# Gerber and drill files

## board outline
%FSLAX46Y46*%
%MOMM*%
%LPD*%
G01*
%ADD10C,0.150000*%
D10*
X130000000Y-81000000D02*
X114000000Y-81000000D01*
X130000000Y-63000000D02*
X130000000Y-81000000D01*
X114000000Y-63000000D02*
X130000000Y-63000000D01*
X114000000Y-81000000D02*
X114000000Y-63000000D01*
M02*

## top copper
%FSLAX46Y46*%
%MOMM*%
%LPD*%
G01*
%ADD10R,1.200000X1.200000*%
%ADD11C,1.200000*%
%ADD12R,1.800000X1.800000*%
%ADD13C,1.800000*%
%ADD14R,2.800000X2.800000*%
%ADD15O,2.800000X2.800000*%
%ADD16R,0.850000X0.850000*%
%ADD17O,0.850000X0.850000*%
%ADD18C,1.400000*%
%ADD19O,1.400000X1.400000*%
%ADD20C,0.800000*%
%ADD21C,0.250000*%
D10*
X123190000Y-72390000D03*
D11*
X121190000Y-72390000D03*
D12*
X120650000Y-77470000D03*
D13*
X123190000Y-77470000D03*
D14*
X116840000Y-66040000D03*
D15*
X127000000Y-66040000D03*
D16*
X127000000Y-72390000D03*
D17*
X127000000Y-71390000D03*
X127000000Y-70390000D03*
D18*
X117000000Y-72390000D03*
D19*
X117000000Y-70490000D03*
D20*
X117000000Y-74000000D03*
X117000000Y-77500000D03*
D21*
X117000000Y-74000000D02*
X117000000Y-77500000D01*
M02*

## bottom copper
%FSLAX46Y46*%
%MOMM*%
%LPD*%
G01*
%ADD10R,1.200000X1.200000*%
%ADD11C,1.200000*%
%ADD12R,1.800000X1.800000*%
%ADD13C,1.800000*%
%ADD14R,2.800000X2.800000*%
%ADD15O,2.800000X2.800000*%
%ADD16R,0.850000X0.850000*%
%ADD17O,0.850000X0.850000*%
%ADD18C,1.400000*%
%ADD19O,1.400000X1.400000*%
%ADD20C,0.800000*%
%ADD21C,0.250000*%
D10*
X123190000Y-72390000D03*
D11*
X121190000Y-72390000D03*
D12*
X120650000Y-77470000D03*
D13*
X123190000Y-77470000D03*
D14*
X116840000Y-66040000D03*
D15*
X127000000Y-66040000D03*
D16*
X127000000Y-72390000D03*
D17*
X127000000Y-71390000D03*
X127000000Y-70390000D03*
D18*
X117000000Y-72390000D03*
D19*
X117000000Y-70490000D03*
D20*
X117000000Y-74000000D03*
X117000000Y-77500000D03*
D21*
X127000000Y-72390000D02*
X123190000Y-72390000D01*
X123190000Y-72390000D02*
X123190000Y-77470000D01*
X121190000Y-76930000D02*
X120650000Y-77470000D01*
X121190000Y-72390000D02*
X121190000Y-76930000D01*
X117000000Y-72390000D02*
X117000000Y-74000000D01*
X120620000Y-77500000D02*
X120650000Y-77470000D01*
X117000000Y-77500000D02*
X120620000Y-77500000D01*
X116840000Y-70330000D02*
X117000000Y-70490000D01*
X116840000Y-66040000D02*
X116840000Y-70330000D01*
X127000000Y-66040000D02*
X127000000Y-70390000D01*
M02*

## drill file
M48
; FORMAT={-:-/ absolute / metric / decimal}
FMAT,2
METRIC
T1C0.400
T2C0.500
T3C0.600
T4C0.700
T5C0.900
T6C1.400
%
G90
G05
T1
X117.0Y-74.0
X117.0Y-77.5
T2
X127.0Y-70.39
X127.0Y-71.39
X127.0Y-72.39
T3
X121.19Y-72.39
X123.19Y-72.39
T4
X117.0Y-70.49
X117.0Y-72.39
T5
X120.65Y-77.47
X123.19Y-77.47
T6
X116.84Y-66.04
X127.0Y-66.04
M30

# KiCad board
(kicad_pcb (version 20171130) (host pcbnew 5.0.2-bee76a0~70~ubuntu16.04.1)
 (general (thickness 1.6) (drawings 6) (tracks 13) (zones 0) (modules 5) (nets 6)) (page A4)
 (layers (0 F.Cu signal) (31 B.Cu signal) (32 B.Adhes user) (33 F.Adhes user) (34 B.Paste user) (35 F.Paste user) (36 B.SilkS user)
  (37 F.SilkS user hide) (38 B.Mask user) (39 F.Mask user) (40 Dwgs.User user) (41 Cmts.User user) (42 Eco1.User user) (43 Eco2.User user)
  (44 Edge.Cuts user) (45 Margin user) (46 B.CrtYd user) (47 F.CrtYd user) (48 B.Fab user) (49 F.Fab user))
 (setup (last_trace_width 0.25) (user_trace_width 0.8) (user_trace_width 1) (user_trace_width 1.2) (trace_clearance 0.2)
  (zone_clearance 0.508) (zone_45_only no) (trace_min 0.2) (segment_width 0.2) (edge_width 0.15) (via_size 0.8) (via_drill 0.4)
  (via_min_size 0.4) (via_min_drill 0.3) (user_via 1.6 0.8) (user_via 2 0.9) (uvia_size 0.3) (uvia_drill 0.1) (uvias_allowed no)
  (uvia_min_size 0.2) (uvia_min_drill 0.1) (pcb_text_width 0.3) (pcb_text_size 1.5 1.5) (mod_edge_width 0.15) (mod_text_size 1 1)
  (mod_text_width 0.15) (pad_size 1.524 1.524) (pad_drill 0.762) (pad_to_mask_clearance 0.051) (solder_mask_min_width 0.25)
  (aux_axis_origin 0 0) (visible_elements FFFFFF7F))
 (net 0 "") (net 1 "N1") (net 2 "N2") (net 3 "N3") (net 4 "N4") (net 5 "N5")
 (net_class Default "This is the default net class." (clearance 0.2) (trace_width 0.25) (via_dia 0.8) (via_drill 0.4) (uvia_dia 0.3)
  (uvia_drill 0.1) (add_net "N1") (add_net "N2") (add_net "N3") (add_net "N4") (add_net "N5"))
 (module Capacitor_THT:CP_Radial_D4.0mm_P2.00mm (layer F.Cu) (at 123.19 72.39 180)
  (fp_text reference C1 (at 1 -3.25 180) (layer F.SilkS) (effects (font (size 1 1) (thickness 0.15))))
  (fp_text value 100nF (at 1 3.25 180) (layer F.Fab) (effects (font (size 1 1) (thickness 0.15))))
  (pad 1 thru_hole rect (at 0 0 180) (size 1.2 1.2) (drill 0.6) (layers *.Cu *.Mask) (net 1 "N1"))
  (pad 2 thru_hole circle (at 2 0 180) (size 1.2 1.2) (drill 0.6) (layers *.Cu *.Mask) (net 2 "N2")))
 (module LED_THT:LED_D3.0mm (layer F.Cu) (at 120.65 77.47)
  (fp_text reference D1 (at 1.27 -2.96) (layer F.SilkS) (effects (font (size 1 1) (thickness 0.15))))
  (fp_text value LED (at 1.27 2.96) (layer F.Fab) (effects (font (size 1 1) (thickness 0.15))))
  (pad 1 thru_hole rect (at 0 0) (size 1.8 1.8) (drill 0.9) (layers *.Cu *.Mask) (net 2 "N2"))
  (pad 2 thru_hole circle (at 2.54 0) (size 1.8 1.8) (drill 0.9) (layers *.Cu *.Mask) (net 1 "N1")))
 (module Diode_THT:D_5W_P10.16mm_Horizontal (layer F.Cu) (at 116.84 66.04)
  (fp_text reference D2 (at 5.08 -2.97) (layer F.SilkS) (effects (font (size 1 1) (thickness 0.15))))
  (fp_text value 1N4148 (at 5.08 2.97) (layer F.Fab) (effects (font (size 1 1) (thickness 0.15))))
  (pad 1 thru_hole rect (at 0 0) (size 2.8 2.8) (drill 1.4) (layers *.Cu *.Mask) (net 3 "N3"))
  (pad 2 thru_hole oval (at 10.16 0) (size 2.8 2.8) (drill 1.4) (layers *.Cu *.Mask) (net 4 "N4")))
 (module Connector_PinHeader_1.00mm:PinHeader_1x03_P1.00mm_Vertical (layer F.Cu) (at 127 72.39 180)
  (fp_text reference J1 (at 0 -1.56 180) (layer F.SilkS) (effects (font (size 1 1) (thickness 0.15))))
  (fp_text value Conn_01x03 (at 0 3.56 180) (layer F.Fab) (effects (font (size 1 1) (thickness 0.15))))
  (pad 1 thru_hole rect (at 0 0 180) (size 0.85 0.85) (drill 0.5) (layers *.Cu *.Mask) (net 1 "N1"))
  (pad 2 thru_hole oval (at 0 1 180) (size 0.85 0.85) (drill 0.5) (layers *.Cu *.Mask) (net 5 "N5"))
  (pad 3 thru_hole oval (at 0 2 180) (size 0.85 0.85) (drill 0.5) (layers *.Cu *.Mask) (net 4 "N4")))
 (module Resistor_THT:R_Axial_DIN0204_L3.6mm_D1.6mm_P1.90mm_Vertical (layer F.Cu) (at 117 72.39 90)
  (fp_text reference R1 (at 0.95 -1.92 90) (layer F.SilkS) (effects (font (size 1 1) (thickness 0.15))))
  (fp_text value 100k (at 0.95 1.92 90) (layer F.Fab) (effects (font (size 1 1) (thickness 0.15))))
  (pad 1 thru_hole circle (at 0 0 90) (size 1.4 1.4) (drill 0.7) (layers *.Cu *.Mask) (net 2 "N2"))
  (pad 2 thru_hole oval (at 1.9 0 90) (size 1.4 1.4) (drill 0.7) (layers *.Cu *.Mask) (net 3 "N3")))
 (gr_line (start 130 81) (end 114 81) (layer Edge.Cuts) (width 0.15))
 (gr_line (start 130 63) (end 130 81) (layer Edge.Cuts) (width 0.15))
 (gr_line (start 114 63) (end 130 63) (layer Edge.Cuts) (width 0.15))
 (gr_line (start 114 81) (end 114 63) (layer Edge.Cuts) (width 0.15))
 (segment (start 127 72.39) (end 123.19 72.39) (width 0.25) (layer B.Cu) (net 1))
 (segment (start 123.19 72.39) (end 123.19 77.47) (width 0.25) (layer B.Cu) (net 1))
 (segment (start 121.19 76.93) (end 120.65 77.47) (width 0.25) (layer B.Cu) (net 2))
 (segment (start 121.19 72.39) (end 121.19 76.93) (width 0.25) (layer B.Cu) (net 2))
 (via (at 117 74) (size 0.8) (drill 0.4) (layers F.Cu B.Cu) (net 2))
 (segment (start 117 72.39) (end 117 74) (width 0.25) (layer B.Cu) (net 2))
 (via (at 117 77.5) (size 0.8) (drill 0.4) (layers F.Cu B.Cu) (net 2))
 (segment (start 117 74) (end 117 77.5) (width 0.25) (layer F.Cu) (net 2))
 (segment (start 120.62 77.5) (end 120.65 77.47) (width 0.25) (layer B.Cu) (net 2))
 (segment (start 117 77.5) (end 120.62 77.5) (width 0.25) (layer B.Cu) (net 2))
 (segment (start 116.84 70.33) (end 117 70.49) (width 0.25) (layer B.Cu) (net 3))
 (segment (start 116.84 66.04) (end 116.84 70.33) (width 0.25) (layer B.Cu) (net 3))
 (segment (start 127 66.04) (end 127 70.39) (width 0.25) (layer B.Cu) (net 4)))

